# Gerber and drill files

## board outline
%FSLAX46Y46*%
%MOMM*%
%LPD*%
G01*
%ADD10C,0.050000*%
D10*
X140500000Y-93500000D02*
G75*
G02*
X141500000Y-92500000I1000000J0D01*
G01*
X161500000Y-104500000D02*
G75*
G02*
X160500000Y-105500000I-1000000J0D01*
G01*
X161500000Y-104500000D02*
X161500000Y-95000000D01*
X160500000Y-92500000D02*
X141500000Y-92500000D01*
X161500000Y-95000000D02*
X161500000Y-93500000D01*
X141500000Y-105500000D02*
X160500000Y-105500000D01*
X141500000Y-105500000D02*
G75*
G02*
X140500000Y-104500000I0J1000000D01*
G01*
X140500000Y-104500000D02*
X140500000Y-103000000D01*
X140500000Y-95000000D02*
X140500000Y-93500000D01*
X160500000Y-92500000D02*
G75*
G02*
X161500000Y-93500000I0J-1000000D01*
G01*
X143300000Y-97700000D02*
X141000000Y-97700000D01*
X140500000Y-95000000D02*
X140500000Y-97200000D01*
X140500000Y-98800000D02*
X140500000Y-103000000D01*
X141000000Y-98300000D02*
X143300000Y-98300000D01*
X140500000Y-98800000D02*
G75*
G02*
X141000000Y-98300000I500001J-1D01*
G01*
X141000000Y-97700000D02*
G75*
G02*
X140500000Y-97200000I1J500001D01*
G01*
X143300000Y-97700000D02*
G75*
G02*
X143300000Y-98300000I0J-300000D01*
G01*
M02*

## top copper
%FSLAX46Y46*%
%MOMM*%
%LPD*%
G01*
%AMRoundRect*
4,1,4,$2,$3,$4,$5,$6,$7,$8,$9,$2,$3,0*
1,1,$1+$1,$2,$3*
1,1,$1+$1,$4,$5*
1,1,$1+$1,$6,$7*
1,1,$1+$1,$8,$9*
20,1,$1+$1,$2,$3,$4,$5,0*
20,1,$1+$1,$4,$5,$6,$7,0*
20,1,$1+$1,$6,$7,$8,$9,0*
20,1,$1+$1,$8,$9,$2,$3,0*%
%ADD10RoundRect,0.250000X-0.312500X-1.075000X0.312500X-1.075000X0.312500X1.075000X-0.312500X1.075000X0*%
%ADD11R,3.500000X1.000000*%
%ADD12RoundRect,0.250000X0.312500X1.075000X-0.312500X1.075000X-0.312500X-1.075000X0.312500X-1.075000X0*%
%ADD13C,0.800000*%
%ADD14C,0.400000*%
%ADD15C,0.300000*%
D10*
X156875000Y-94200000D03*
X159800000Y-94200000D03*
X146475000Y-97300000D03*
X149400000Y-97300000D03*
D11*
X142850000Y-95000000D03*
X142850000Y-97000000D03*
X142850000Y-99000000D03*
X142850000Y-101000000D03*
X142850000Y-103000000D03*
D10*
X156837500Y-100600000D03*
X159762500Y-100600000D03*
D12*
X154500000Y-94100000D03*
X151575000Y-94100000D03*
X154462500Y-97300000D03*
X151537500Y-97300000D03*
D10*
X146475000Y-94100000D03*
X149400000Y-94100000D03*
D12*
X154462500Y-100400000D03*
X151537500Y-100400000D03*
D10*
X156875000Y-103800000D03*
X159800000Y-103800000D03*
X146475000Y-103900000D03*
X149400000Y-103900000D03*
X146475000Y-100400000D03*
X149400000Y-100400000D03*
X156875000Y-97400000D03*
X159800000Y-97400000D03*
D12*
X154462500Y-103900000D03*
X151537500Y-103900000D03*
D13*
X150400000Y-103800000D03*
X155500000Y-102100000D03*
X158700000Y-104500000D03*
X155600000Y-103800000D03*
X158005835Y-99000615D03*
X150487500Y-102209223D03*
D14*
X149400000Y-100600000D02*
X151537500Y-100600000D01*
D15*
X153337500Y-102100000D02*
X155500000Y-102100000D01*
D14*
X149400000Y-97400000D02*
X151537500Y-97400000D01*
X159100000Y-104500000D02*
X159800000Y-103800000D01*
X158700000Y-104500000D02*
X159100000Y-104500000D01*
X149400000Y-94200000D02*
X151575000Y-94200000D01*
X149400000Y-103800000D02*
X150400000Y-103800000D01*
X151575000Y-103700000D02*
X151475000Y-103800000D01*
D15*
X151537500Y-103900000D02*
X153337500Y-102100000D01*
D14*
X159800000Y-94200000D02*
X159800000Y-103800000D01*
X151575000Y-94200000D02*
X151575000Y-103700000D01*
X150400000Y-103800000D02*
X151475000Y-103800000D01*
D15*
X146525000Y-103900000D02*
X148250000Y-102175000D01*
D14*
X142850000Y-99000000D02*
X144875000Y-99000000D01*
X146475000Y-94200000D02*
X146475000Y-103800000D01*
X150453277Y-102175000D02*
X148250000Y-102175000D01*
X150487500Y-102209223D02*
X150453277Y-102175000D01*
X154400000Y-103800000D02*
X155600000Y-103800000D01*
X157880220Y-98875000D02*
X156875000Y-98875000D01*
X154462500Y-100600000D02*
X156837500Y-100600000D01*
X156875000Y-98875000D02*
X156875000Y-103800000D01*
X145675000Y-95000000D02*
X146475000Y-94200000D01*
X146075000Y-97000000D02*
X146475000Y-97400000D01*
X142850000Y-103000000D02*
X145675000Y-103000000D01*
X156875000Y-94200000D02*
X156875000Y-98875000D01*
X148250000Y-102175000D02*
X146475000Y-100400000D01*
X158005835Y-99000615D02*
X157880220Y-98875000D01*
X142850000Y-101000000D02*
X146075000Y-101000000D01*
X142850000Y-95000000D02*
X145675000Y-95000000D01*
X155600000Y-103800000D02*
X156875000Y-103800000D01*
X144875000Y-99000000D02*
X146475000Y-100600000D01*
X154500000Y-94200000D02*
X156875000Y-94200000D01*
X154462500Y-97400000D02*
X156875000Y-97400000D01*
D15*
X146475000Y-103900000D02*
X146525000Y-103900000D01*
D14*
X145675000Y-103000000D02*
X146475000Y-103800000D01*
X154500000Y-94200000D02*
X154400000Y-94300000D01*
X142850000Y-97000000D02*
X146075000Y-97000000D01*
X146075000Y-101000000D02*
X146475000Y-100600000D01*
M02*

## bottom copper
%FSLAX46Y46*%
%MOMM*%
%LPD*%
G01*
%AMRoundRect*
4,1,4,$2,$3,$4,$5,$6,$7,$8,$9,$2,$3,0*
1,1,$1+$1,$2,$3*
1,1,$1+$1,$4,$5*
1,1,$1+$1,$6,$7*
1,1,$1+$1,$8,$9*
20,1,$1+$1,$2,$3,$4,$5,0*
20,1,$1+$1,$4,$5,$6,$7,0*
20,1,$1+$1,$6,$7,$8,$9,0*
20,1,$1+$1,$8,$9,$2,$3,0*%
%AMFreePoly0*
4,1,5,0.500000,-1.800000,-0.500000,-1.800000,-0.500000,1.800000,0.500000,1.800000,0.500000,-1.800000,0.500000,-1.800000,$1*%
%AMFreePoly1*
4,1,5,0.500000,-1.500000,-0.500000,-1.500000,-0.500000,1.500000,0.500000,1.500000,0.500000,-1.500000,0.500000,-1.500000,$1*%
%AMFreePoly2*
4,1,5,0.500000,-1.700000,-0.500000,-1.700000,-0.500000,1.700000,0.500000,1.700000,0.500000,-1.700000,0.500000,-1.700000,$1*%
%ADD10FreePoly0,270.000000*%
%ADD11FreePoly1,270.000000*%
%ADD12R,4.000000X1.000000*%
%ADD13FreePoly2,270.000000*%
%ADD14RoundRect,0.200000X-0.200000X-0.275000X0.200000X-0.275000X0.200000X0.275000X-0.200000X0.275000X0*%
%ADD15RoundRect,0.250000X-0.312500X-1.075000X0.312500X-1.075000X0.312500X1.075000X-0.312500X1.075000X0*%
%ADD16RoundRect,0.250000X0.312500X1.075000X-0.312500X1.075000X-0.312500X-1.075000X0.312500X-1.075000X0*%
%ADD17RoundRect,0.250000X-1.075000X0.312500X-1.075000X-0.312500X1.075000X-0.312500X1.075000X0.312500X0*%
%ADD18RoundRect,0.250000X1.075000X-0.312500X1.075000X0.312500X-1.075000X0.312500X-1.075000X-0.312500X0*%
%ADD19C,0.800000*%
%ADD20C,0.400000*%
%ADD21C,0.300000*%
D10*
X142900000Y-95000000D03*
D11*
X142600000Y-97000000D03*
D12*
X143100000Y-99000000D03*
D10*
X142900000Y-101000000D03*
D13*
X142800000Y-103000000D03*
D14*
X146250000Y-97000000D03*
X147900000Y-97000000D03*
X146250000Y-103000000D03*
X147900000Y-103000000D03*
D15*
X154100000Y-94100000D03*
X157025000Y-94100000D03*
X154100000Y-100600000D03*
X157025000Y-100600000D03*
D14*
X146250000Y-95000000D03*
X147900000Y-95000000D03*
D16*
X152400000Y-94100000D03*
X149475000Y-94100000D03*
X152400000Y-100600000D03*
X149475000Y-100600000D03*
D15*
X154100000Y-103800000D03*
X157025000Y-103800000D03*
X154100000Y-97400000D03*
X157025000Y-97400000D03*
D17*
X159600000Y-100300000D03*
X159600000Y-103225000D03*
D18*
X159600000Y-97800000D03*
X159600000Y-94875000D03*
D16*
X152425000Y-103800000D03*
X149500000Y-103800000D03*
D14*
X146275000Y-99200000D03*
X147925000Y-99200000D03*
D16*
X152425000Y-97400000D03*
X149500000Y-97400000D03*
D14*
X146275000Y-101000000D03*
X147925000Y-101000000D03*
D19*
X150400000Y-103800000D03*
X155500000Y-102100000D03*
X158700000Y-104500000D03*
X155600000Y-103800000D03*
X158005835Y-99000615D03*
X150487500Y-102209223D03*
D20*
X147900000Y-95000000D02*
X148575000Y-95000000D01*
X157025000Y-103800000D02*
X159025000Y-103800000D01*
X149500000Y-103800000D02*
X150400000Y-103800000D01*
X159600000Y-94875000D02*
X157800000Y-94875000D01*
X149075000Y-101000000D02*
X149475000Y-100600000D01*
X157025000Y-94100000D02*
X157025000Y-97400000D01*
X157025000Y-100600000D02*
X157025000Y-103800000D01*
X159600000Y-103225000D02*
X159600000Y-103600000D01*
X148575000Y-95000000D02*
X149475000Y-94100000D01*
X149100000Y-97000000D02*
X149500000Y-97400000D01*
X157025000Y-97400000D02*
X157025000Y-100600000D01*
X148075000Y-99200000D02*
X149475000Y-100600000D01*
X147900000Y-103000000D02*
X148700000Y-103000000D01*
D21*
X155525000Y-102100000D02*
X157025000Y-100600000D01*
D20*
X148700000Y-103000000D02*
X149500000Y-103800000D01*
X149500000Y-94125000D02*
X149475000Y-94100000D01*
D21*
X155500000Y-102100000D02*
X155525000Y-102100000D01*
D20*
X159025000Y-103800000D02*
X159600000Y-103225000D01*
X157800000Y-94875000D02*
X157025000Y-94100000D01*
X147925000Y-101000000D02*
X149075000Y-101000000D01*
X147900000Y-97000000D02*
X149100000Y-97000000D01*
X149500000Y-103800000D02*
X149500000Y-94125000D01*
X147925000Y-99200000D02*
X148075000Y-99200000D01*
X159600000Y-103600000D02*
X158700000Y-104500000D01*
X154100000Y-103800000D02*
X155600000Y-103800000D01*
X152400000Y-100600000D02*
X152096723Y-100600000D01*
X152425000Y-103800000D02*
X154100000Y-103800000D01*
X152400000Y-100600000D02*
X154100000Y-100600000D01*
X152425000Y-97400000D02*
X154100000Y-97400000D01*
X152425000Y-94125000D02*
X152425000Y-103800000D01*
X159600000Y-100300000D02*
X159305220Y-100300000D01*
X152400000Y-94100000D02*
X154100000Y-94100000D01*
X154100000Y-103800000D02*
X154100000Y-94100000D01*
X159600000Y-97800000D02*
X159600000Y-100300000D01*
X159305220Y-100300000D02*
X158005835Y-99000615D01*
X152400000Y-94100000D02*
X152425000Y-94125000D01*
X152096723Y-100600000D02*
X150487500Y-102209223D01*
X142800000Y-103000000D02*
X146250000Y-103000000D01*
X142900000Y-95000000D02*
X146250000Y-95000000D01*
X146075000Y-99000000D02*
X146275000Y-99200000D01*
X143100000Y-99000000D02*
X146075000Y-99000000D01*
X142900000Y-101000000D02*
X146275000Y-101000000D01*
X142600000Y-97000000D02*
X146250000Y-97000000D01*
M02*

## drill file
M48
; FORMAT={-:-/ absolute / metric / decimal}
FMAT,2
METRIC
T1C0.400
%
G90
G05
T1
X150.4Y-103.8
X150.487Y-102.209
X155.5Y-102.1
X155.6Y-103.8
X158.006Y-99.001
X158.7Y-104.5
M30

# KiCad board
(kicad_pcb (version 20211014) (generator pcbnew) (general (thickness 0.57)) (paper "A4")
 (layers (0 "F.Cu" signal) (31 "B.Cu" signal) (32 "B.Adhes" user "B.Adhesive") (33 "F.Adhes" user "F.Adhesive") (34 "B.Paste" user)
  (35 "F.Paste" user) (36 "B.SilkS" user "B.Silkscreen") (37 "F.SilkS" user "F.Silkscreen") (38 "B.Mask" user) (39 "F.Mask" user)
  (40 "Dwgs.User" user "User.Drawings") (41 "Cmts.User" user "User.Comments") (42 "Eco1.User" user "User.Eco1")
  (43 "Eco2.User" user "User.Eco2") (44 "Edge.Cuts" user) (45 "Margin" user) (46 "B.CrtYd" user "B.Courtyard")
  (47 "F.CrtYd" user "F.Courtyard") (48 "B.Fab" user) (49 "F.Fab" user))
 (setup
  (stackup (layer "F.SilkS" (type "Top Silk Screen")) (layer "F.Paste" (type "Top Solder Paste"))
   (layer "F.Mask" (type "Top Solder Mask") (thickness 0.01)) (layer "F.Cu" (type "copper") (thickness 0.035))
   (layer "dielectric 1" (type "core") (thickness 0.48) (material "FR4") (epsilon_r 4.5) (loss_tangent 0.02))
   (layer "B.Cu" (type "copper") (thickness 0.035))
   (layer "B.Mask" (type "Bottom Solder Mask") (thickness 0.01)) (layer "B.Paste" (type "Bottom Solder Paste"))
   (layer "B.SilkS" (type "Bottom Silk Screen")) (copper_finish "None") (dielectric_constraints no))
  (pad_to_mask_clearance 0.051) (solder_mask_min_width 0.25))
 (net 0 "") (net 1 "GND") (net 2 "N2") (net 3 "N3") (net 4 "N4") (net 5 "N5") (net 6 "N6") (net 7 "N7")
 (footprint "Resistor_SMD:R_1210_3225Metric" (layer "F.Cu") (at 158.3375 94.2)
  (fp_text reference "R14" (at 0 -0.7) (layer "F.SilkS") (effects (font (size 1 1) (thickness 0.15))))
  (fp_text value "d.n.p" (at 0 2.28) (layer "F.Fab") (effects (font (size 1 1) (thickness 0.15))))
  (pad "1" smd roundrect (at -1.4625 0) (size 1.125 2.65) (layers "F.Cu" "F.Paste" "F.Mask") (roundrect_rratio 0.222222) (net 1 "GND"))
  (pad "2" smd roundrect (at 1.4625 0) (size 1.125 2.65) (layers "F.Cu" "F.Paste" "F.Mask") (roundrect_rratio 0.222222) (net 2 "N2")))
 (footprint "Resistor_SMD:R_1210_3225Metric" (layer "F.Cu") (at 147.9375 97.3)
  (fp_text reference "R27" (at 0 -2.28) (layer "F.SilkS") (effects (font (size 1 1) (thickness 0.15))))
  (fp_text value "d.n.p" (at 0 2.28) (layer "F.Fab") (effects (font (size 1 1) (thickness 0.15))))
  (pad "1" smd roundrect (at -1.4625 0) (size 1.125 2.65) (layers "F.Cu" "F.Paste" "F.Mask") (roundrect_rratio 0.222222) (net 1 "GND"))
  (pad "2" smd roundrect (at 1.4625 0) (size 1.125 2.65) (layers "F.Cu" "F.Paste" "F.Mask") (roundrect_rratio 0.222222) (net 2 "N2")))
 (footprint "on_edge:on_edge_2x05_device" (layer "F.Cu") (at 140.5 99 -90)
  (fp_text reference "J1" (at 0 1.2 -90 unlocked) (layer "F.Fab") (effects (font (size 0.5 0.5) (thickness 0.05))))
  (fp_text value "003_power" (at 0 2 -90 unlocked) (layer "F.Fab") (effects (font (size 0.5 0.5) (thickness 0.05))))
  (fp_line (start -1.3 -2.8) (end -1.3 -0.5) (layer "Edge.Cuts") (width 0.05))
  (fp_line (start -4 0) (end -1.8 0) (layer "Edge.Cuts") (width 0.05))
  (fp_line (start -0.2 0) (end 4 0) (layer "Edge.Cuts") (width 0.05))
  (fp_line (start -0.7 -0.5) (end -0.7 -2.8) (layer "Edge.Cuts") (width 0.05))
  (fp_arc (start -0.2 0) (mid -0.553553 -0.146447) (end -0.7 -0.5) (layer "Edge.Cuts") (width 0.05))
  (fp_arc (start -1.3 -0.5) (mid -1.446447 -0.146447) (end -1.8 0) (layer "Edge.Cuts") (width 0.05))
  (fp_arc (start -1.3 -2.8) (mid -1 -3.1) (end -0.7 -2.8) (layer "Edge.Cuts") (width 0.05))
  (pad "1" smd rect (at -4 -2.35 90) (size 1 3.5) (layers "F.Cu" "F.Mask") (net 1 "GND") (zone_connect 0))
  (pad "2" smd rect (at -2 -2.35 270) (size 1 3.5) (layers "F.Cu" "F.Mask") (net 1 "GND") (zone_connect 0))
  (pad "3" smd rect (at 0 -2.35 270) (size 1 3.5) (layers "F.Cu" "F.Mask") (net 1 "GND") (zone_connect 0))
  (pad "4" smd rect (at 2 -2.35 90) (size 1 3.5) (layers "F.Cu" "F.Mask") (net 1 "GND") (zone_connect 0))
  (pad "5" smd rect (at 4 -2.35 90) (size 1 3.5) (layers "F.Cu" "F.Mask") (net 1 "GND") (zone_connect 0))
  (pad "6" smd custom (at -4 -2.4 270) (size 1 3.6) (layers "B.Cu" "B.Mask") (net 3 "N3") (zone_connect 0)
   (options (clearance outline) (anchor rect)) (primitives))
  (pad "7" smd custom (at -2 -2.1 270) (size 1 3) (layers "B.Cu" "B.Mask") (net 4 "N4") (zone_connect 0)
   (options (clearance outline) (anchor rect)) (primitives))
  (pad "8" smd rect (at 0 -2.6 270) (size 1 4) (layers "B.Cu" "B.Mask") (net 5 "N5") (zone_connect 0))
  (pad "9" smd custom (at 2 -2.4 270) (size 1 3.6) (layers "B.Cu" "B.Mask") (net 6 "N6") (zone_connect 0)
   (options (clearance outline) (anchor rect)) (primitives))
  (pad "10" smd custom (at 4 -2.3 270) (size 1 3.4) (layers "B.Cu" "B.Mask") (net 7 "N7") (zone_connect 0)
   (options (clearance outline) (anchor rect)) (primitives)))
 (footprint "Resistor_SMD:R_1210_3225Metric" (layer "F.Cu") (at 158.3 100.6)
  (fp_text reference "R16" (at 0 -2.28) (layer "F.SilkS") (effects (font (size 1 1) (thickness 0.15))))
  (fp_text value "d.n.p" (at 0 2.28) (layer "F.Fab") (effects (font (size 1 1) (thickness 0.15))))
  (pad "1" smd roundrect (at -1.4625 0) (size 1.125 2.65) (layers "F.Cu" "F.Paste" "F.Mask") (roundrect_rratio 0.222222) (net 1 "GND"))
  (pad "2" smd roundrect (at 1.4625 0) (size 1.125 2.65) (layers "F.Cu" "F.Paste" "F.Mask") (roundrect_rratio 0.222222) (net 2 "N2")))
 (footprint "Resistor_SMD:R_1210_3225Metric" (layer "F.Cu") (at 153.0375 94.1 180)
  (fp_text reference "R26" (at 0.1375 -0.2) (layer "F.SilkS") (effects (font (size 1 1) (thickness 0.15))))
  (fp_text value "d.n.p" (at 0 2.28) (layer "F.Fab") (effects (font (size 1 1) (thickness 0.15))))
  (pad "1" smd roundrect (at -1.4625 0 180) (size 1.125 2.65) (layers "F.Cu" "F.Paste" "F.Mask") (roundrect_rratio 0.222222) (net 1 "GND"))
  (pad "2" smd roundrect (at 1.4625 0 180) (size 1.125 2.65) (layers "F.Cu" "F.Paste" "F.Mask") (roundrect_rratio 0.222222) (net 2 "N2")))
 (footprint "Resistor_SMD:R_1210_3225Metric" (layer "F.Cu") (at 153 97.3 180)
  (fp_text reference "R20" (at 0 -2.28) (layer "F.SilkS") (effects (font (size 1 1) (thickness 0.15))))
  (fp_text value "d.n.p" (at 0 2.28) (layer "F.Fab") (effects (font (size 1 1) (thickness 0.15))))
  (pad "1" smd roundrect (at -1.4625 0 180) (size 1.125 2.65) (layers "F.Cu" "F.Paste" "F.Mask") (roundrect_rratio 0.222222) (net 1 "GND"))
  (pad "2" smd roundrect (at 1.4625 0 180) (size 1.125 2.65) (layers "F.Cu" "F.Paste" "F.Mask") (roundrect_rratio 0.222222) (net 2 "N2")))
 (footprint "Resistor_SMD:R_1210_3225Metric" (layer "F.Cu") (at 147.9375 94.1)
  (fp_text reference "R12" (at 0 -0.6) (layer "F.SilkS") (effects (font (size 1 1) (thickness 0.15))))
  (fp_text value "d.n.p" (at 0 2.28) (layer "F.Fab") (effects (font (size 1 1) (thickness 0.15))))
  (pad "1" smd roundrect (at -1.4625 0) (size 1.125 2.65) (layers "F.Cu" "F.Paste" "F.Mask") (roundrect_rratio 0.222222) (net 1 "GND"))
  (pad "2" smd roundrect (at 1.4625 0) (size 1.125 2.65) (layers "F.Cu" "F.Paste" "F.Mask") (roundrect_rratio 0.222222) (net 2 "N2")))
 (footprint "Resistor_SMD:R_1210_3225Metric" (layer "F.Cu") (at 153 100.4 180)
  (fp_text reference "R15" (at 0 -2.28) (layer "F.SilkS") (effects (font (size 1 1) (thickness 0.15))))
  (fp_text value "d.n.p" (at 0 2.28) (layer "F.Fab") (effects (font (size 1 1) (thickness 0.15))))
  (pad "1" smd roundrect (at -1.4625 0 180) (size 1.125 2.65) (layers "F.Cu" "F.Paste" "F.Mask") (roundrect_rratio 0.222222) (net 1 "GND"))
  (pad "2" smd roundrect (at 1.4625 0 180) (size 1.125 2.65) (layers "F.Cu" "F.Paste" "F.Mask") (roundrect_rratio 0.222222) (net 2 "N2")))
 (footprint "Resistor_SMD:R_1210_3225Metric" (layer "F.Cu") (at 158.3375 103.8)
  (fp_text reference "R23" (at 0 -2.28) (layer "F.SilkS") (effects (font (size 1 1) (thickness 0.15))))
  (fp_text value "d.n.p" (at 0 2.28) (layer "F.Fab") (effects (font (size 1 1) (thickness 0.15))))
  (pad "1" smd roundrect (at -1.4625 0) (size 1.125 2.65) (layers "F.Cu" "F.Paste" "F.Mask") (roundrect_rratio 0.222222) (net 1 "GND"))
  (pad "2" smd roundrect (at 1.4625 0) (size 1.125 2.65) (layers "F.Cu" "F.Paste" "F.Mask") (roundrect_rratio 0.222222) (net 2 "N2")))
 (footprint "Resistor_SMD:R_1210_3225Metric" (layer "F.Cu") (at 147.9375 103.9)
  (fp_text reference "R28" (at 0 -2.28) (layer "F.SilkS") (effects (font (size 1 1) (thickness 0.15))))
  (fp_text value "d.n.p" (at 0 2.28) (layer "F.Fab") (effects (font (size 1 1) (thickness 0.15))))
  (pad "1" smd roundrect (at -1.4625 0) (size 1.125 2.65) (layers "F.Cu" "F.Paste" "F.Mask") (roundrect_rratio 0.222222) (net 1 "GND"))
  (pad "2" smd roundrect (at 1.4625 0) (size 1.125 2.65) (layers "F.Cu" "F.Paste" "F.Mask") (roundrect_rratio 0.222222) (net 2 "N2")))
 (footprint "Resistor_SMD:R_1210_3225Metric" (layer "F.Cu") (at 147.9375 100.4)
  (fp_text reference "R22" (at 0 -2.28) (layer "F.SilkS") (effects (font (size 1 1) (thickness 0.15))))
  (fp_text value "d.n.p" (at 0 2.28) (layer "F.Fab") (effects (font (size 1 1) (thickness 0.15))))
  (pad "1" smd roundrect (at -1.4625 0) (size 1.125 2.65) (layers "F.Cu" "F.Paste" "F.Mask") (roundrect_rratio 0.222222) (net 1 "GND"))
  (pad "2" smd roundrect (at 1.4625 0) (size 1.125 2.65) (layers "F.Cu" "F.Paste" "F.Mask") (roundrect_rratio 0.222222) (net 2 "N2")))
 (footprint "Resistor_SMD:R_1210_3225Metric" (layer "F.Cu") (at 158.3375 97.4)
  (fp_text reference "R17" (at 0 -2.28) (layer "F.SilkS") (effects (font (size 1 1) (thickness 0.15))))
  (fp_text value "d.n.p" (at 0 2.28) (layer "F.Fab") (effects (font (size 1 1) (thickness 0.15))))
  (pad "1" smd roundrect (at -1.4625 0) (size 1.125 2.65) (layers "F.Cu" "F.Paste" "F.Mask") (roundrect_rratio 0.222222) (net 1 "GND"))
  (pad "2" smd roundrect (at 1.4625 0) (size 1.125 2.65) (layers "F.Cu" "F.Paste" "F.Mask") (roundrect_rratio 0.222222) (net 2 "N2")))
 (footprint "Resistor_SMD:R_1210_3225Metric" (layer "F.Cu") (at 153 103.9 180)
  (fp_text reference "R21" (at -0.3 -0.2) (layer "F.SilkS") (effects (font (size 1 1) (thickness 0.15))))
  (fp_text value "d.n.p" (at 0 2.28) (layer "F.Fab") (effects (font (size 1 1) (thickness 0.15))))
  (pad "1" smd roundrect (at -1.4625 0 180) (size 1.125 2.65) (layers "F.Cu" "F.Paste" "F.Mask") (roundrect_rratio 0.222222) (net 1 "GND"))
  (pad "2" smd roundrect (at 1.4625 0 180) (size 1.125 2.65) (layers "F.Cu" "F.Paste" "F.Mask") (roundrect_rratio 0.222222) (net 2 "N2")))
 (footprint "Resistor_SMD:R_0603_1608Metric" (layer "B.Cu") (at 147.075 97)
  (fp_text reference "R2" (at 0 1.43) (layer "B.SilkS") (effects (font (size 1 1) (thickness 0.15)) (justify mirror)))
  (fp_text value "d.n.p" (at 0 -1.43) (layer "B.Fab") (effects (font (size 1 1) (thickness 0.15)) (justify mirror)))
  (pad "1" smd roundrect (at -0.825 0) (size 0.8 0.95) (layers "B.Cu" "B.Paste" "B.Mask") (roundrect_rratio 0.25) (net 4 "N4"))
  (pad "2" smd roundrect (at 0.825 0) (size 0.8 0.95) (layers "B.Cu" "B.Paste" "B.Mask") (roundrect_rratio 0.25) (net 2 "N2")))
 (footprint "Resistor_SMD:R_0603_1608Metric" (layer "B.Cu") (at 147.075 103)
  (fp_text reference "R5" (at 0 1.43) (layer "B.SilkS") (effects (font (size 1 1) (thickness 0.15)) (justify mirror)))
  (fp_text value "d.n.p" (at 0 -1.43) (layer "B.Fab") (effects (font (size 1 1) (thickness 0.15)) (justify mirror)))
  (pad "1" smd roundrect (at -0.825 0) (size 0.8 0.95) (layers "B.Cu" "B.Paste" "B.Mask") (roundrect_rratio 0.25) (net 7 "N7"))
  (pad "2" smd roundrect (at 0.825 0) (size 0.8 0.95) (layers "B.Cu" "B.Paste" "B.Mask") (roundrect_rratio 0.25) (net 2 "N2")))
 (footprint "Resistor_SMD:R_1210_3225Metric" (layer "B.Cu") (at 155.5625 94.1)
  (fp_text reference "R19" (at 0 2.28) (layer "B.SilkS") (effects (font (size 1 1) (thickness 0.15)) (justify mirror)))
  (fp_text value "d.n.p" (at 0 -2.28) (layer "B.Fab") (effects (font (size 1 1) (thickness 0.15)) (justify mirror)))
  (pad "1" smd roundrect (at -1.4625 0) (size 1.125 2.65) (layers "B.Cu" "B.Paste" "B.Mask") (roundrect_rratio 0.222222) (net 1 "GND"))
  (pad "2" smd roundrect (at 1.4625 0) (size 1.125 2.65) (layers "B.Cu" "B.Paste" "B.Mask") (roundrect_rratio 0.222222) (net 2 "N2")))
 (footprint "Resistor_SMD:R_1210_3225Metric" (layer "B.Cu") (at 155.5625 100.6)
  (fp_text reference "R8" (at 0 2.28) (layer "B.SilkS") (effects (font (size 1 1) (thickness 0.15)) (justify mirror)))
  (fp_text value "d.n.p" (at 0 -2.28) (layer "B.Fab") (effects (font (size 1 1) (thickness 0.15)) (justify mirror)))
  (pad "1" smd roundrect (at -1.4625 0) (size 1.125 2.65) (layers "B.Cu" "B.Paste" "B.Mask") (roundrect_rratio 0.222222) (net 1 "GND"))
  (pad "2" smd roundrect (at 1.4625 0) (size 1.125 2.65) (layers "B.Cu" "B.Paste" "B.Mask") (roundrect_rratio 0.222222) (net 2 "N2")))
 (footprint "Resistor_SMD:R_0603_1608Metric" (layer "B.Cu") (at 147.075 95)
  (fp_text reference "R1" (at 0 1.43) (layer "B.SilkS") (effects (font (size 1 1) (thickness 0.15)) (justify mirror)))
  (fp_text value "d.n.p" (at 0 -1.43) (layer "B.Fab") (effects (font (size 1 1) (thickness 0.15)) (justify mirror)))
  (pad "1" smd roundrect (at -0.825 0) (size 0.8 0.95) (layers "B.Cu" "B.Paste" "B.Mask") (roundrect_rratio 0.25) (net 3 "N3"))
  (pad "2" smd roundrect (at 0.825 0) (size 0.8 0.95) (layers "B.Cu" "B.Paste" "B.Mask") (roundrect_rratio 0.25) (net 2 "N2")))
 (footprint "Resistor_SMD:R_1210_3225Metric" (layer "B.Cu") (at 150.9375 94.1 180)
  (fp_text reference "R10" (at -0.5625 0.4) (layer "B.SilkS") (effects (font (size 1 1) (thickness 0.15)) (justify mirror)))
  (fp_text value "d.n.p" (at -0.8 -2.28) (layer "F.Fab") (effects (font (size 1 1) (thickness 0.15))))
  (pad "1" smd roundrect (at -1.4625 0 180) (size 1.125 2.65) (layers "B.Cu" "B.Paste" "B.Mask") (roundrect_rratio 0.222222) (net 1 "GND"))
  (pad "2" smd roundrect (at 1.4625 0 180) (size 1.125 2.65) (layers "B.Cu" "B.Paste" "B.Mask") (roundrect_rratio 0.222222) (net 2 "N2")))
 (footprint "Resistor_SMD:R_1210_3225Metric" (layer "B.Cu") (at 150.9375 100.6 180)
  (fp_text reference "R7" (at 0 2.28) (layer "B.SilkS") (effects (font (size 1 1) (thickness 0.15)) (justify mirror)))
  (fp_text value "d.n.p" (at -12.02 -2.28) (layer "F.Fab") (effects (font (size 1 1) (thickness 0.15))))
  (pad "1" smd roundrect (at -1.4625 0 180) (size 1.125 2.65) (layers "B.Cu" "B.Paste" "B.Mask") (roundrect_rratio 0.222222) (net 1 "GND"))
  (pad "2" smd roundrect (at 1.4625 0 180) (size 1.125 2.65) (layers "B.Cu" "B.Paste" "B.Mask") (roundrect_rratio 0.222222) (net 2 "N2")))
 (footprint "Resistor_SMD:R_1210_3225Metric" (layer "B.Cu") (at 155.5625 103.8)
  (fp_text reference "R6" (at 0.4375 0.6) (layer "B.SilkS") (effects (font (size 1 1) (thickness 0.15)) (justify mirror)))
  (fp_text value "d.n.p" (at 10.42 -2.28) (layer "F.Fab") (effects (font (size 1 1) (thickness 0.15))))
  (pad "1" smd roundrect (at -1.4625 0) (size 1.125 2.65) (layers "B.Cu" "B.Paste" "B.Mask") (roundrect_rratio 0.222222) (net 1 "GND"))
  (pad "2" smd roundrect (at 1.4625 0) (size 1.125 2.65) (layers "B.Cu" "B.Paste" "B.Mask") (roundrect_rratio 0.222222) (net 2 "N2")))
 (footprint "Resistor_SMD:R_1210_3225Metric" (layer "B.Cu") (at 155.5625 97.4)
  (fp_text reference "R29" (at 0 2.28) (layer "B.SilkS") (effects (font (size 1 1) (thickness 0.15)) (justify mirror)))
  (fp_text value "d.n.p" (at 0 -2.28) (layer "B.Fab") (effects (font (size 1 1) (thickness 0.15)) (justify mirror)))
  (pad "1" smd roundrect (at -1.4625 0) (size 1.125 2.65) (layers "B.Cu" "B.Paste" "B.Mask") (roundrect_rratio 0.222222) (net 1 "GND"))
  (pad "2" smd roundrect (at 1.4625 0) (size 1.125 2.65) (layers "B.Cu" "B.Paste" "B.Mask") (roundrect_rratio 0.222222) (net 2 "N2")))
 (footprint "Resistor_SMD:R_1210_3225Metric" (layer "B.Cu") (at 159.6 101.7625 -90)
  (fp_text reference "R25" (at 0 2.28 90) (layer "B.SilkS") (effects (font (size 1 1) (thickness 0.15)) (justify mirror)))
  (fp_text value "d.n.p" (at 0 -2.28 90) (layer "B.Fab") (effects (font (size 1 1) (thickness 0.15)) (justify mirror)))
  (pad "1" smd roundrect (at -1.4625 0 270) (size 1.125 2.65) (layers "B.Cu" "B.Paste" "B.Mask") (roundrect_rratio 0.222222) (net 1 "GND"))
  (pad "2" smd roundrect (at 1.4625 0 270) (size 1.125 2.65) (layers "B.Cu" "B.Paste" "B.Mask") (roundrect_rratio 0.222222) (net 2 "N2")))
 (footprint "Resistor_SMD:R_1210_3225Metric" (layer "B.Cu") (at 159.6 96.3375 90)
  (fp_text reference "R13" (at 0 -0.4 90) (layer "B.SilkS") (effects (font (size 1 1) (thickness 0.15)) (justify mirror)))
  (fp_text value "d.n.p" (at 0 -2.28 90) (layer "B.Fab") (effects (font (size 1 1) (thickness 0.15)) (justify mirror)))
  (pad "1" smd roundrect (at -1.4625 0 90) (size 1.125 2.65) (layers "B.Cu" "B.Paste" "B.Mask") (roundrect_rratio 0.222222) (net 1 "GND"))
  (pad "2" smd roundrect (at 1.4625 0 90) (size 1.125 2.65) (layers "B.Cu" "B.Paste" "B.Mask") (roundrect_rratio 0.222222) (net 2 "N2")))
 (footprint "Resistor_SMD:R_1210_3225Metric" (layer "B.Cu") (at 150.9625 103.8 180)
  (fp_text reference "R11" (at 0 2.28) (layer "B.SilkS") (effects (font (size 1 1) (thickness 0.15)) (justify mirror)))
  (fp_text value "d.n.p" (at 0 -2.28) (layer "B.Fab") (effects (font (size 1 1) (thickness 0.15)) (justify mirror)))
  (pad "1" smd roundrect (at -1.4625 0 180) (size 1.125 2.65) (layers "B.Cu" "B.Paste" "B.Mask") (roundrect_rratio 0.222222) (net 1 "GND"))
  (pad "2" smd roundrect (at 1.4625 0 180) (size 1.125 2.65) (layers "B.Cu" "B.Paste" "B.Mask") (roundrect_rratio 0.222222) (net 2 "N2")))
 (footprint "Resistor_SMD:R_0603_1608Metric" (layer "B.Cu") (at 147.1 99.2)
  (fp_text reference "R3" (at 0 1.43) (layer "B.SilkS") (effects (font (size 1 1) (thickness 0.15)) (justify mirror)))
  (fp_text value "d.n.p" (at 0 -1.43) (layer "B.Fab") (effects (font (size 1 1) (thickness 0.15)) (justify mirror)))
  (pad "1" smd roundrect (at -0.825 0) (size 0.8 0.95) (layers "B.Cu" "B.Paste" "B.Mask") (roundrect_rratio 0.25) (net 5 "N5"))
  (pad "2" smd roundrect (at 0.825 0) (size 0.8 0.95) (layers "B.Cu" "B.Paste" "B.Mask") (roundrect_rratio 0.25) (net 2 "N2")))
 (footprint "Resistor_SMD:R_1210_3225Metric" (layer "B.Cu") (at 150.9625 97.4 180)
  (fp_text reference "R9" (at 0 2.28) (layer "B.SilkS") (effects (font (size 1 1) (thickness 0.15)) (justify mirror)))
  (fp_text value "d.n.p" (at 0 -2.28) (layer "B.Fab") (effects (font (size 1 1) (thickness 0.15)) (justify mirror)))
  (pad "1" smd roundrect (at -1.4625 0 180) (size 1.125 2.65) (layers "B.Cu" "B.Paste" "B.Mask") (roundrect_rratio 0.222222) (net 1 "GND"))
  (pad "2" smd roundrect (at 1.4625 0 180) (size 1.125 2.65) (layers "B.Cu" "B.Paste" "B.Mask") (roundrect_rratio 0.222222) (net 2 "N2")))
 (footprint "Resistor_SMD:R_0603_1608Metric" (layer "B.Cu") (at 147.1 101)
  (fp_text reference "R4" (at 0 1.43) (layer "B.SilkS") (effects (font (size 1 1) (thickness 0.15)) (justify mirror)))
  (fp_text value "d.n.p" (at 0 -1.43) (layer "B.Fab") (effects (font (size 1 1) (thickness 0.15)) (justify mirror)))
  (pad "1" smd roundrect (at -0.825 0) (size 0.8 0.95) (layers "B.Cu" "B.Paste" "B.Mask") (roundrect_rratio 0.25) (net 6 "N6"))
  (pad "2" smd roundrect (at 0.825 0) (size 0.8 0.95) (layers "B.Cu" "B.Paste" "B.Mask") (roundrect_rratio 0.25) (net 2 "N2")))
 (gr_arc (start 140.5 93.5) (mid 140.792893 92.792893) (end 141.5 92.5) (layer "Edge.Cuts") (width 0.05))
 (gr_arc (start 161.5 104.5) (mid 161.207107 105.207107) (end 160.5 105.5) (layer "Edge.Cuts") (width 0.05))
 (gr_line (start 161.5 104.5) (end 161.5 95) (layer "Edge.Cuts") (width 0.05))
 (gr_line (start 160.5 92.5) (end 141.5 92.5) (layer "Edge.Cuts") (width 0.05))
 (gr_line (start 161.5 95) (end 161.5 93.5) (layer "Edge.Cuts") (width 0.05))
 (gr_line (start 141.5 105.5) (end 160.5 105.5) (layer "Edge.Cuts") (width 0.05))
 (gr_arc (start 141.5 105.5) (mid 140.792893 105.207107) (end 140.5 104.5) (layer "Edge.Cuts") (width 0.05))
 (gr_line (start 140.5 104.5) (end 140.5 103) (layer "Edge.Cuts") (width 0.05))
 (gr_line (start 140.5 95) (end 140.5 93.5) (layer "Edge.Cuts") (width 0.05))
 (gr_arc (start 160.5 92.5) (mid 161.207107 92.792893) (end 161.5 93.5) (layer "Edge.Cuts") (width 0.05))
 (segment (start 149.4 100.6) (end 151.5375 100.6) (width 0.4) (layer "F.Cu") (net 2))
 (segment (start 153.3375 102.1) (end 155.5 102.1) (width 0.3) (layer "F.Cu") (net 2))
 (segment (start 149.4 97.4) (end 151.5375 97.4) (width 0.4) (layer "F.Cu") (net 2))
 (segment (start 159.1 104.5) (end 159.8 103.8) (width 0.4) (layer "F.Cu") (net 2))
 (segment (start 158.7 104.5) (end 159.1 104.5) (width 0.4) (layer "F.Cu") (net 2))
 (segment (start 149.4 94.2) (end 151.575 94.2) (width 0.4) (layer "F.Cu") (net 2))
 (segment (start 149.4 103.8) (end 150.4 103.8) (width 0.4) (layer "F.Cu") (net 2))
 (segment (start 151.575 103.7) (end 151.475 103.8) (width 0.4) (layer "F.Cu") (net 2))
 (segment (start 151.5375 103.9) (end 153.3375 102.1) (width 0.3) (layer "F.Cu") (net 2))
 (segment (start 159.8 94.2) (end 159.8 103.8) (width 0.4) (layer "F.Cu") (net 2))
 (segment (start 151.575 94.2) (end 151.575 103.7) (width 0.4) (layer "F.Cu") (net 2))
 (segment (start 150.4 103.8) (end 151.475 103.8) (width 0.4) (layer "F.Cu") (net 2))
 (via (at 150.4 103.8) (size 0.8) (drill 0.4) (layers "F.Cu" "B.Cu") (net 2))
 (via (at 155.5 102.1) (size 0.8) (drill 0.4) (layers "F.Cu" "B.Cu") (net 2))
 (via (at 158.7 104.5) (size 0.8) (drill 0.4) (layers "F.Cu" "B.Cu") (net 2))
 (segment (start 147.9 95) (end 148.575 95) (width 0.4) (layer "B.Cu") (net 2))
 (segment (start 157.025 103.8) (end 159.025 103.8) (width 0.4) (layer "B.Cu") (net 2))
 (segment (start 149.5 103.8) (end 150.4 103.8) (width 0.4) (layer "B.Cu") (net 2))
 (segment (start 159.6 94.875) (end 157.8 94.875) (width 0.4) (layer "B.Cu") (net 2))
 (segment (start 149.075 101) (end 149.475 100.6) (width 0.4) (layer "B.Cu") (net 2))
 (segment (start 157.025 94.1) (end 157.025 97.4) (width 0.4) (layer "B.Cu") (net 2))
 (segment (start 157.025 100.6) (end 157.025 103.8) (width 0.4) (layer "B.Cu") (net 2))
 (segment (start 159.6 103.225) (end 159.6 103.6) (width 0.4) (layer "B.Cu") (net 2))
 (segment (start 148.575 95) (end 149.475 94.1) (width 0.4) (layer "B.Cu") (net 2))
 (segment (start 149.1 97) (end 149.5 97.4) (width 0.4) (layer "B.Cu") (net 2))
 (segment (start 157.025 97.4) (end 157.025 100.6) (width 0.4) (layer "B.Cu") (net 2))
 (segment (start 148.075 99.2) (end 149.475 100.6) (width 0.4) (layer "B.Cu") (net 2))
 (segment (start 147.9 103) (end 148.7 103) (width 0.4) (layer "B.Cu") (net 2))
 (segment (start 155.525 102.1) (end 157.025 100.6) (width 0.3) (layer "B.Cu") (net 2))
 (segment (start 148.7 103) (end 149.5 103.8) (width 0.4) (layer "B.Cu") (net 2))
 (segment (start 149.5 94.125) (end 149.475 94.1) (width 0.4) (layer "B.Cu") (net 2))
 (segment (start 155.5 102.1) (end 155.525 102.1) (width 0.3) (layer "B.Cu") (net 2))
 (segment (start 159.025 103.8) (end 159.6 103.225) (width 0.4) (layer "B.Cu") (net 2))
 (segment (start 157.8 94.875) (end 157.025 94.1) (width 0.4) (layer "B.Cu") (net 2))
 (segment (start 147.925 101) (end 149.075 101) (width 0.4) (layer "B.Cu") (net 2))
 (segment (start 147.9 97) (end 149.1 97) (width 0.4) (layer "B.Cu") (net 2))
 (segment (start 149.5 103.8) (end 149.5 94.125) (width 0.4) (layer "B.Cu") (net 2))
 (segment (start 147.925 99.2) (end 148.075 99.2) (width 0.4) (layer "B.Cu") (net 2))
 (segment (start 159.6 103.6) (end 158.7 104.5) (width 0.4) (layer "B.Cu") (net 2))
 (segment (start 146.525 103.9) (end 148.25 102.175) (width 0.3) (layer "F.Cu") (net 1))
 (segment (start 142.85 99) (end 144.875 99) (width 0.4) (layer "F.Cu") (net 1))
 (segment (start 146.475 94.2) (end 146.475 103.8) (width 0.4) (layer "F.Cu") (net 1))
 (segment (start 150.453277 102.175) (end 148.25 102.175) (width 0.4) (layer "F.Cu") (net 1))
 (segment (start 150.4875 102.209223) (end 150.453277 102.175) (width 0.4) (layer "F.Cu") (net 1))
 (segment (start 154.4 103.8) (end 155.6 103.8) (width 0.4) (layer "F.Cu") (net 1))
 (segment (start 157.88022 98.875) (end 156.875 98.875) (width 0.4) (layer "F.Cu") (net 1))
 (segment (start 154.4625 100.6) (end 156.8375 100.6) (width 0.4) (layer "F.Cu") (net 1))
 (segment (start 156.875 98.875) (end 156.875 103.8) (width 0.4) (layer "F.Cu") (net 1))
 (segment (start 145.675 95) (end 146.475 94.2) (width 0.4) (layer "F.Cu") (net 1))
 (segment (start 146.075 97) (end 146.475 97.4) (width 0.4) (layer "F.Cu") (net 1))
 (segment (start 142.85 103) (end 145.675 103) (width 0.4) (layer "F.Cu") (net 1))
 (segment (start 156.875 94.2) (end 156.875 98.875) (width 0.4) (layer "F.Cu") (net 1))
 (segment (start 148.25 102.175) (end 146.475 100.4) (width 0.4) (layer "F.Cu") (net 1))
 (segment (start 158.005835 99.000615) (end 157.88022 98.875) (width 0.4) (layer "F.Cu") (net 1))
 (segment (start 142.85 101) (end 146.075 101) (width 0.4) (layer "F.Cu") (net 1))
 (segment (start 142.85 95) (end 145.675 95) (width 0.4) (layer "F.Cu") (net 1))
 (segment (start 155.6 103.8) (end 156.875 103.8) (width 0.4) (layer "F.Cu") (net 1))
 (segment (start 144.875 99) (end 146.475 100.6) (width 0.4) (layer "F.Cu") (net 1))
 (segment (start 154.5 94.2) (end 156.875 94.2) (width 0.4) (layer "F.Cu") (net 1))
 (segment (start 154.4625 97.4) (end 156.875 97.4) (width 0.4) (layer "F.Cu") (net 1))
 (segment (start 146.475 103.9) (end 146.525 103.9) (width 0.3) (layer "F.Cu") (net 1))
 (segment (start 145.675 103) (end 146.475 103.8) (width 0.4) (layer "F.Cu") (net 1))
 (segment (start 154.5 94.2) (end 154.4 94.3) (width 0.4) (layer "F.Cu") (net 1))
 (segment (start 142.85 97) (end 146.075 97) (width 0.4) (layer "F.Cu") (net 1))
 (segment (start 146.075 101) (end 146.475 100.6) (width 0.4) (layer "F.Cu") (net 1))
 (via (at 155.6 103.8) (size 0.8) (drill 0.4) (layers "F.Cu" "B.Cu") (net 1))
 (via (at 158.005835 99.000615) (size 0.8) (drill 0.4) (layers "F.Cu" "B.Cu") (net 1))
 (via (at 150.4875 102.209223) (size 0.8) (drill 0.4) (layers "F.Cu" "B.Cu") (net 1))
 (segment (start 154.1 103.8) (end 155.6 103.8) (width 0.4) (layer "B.Cu") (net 1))
 (segment (start 152.4 100.6) (end 152.096723 100.6) (width 0.4) (layer "B.Cu") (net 1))
 (segment (start 152.425 103.8) (end 154.1 103.8) (width 0.4) (layer "B.Cu") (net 1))
 (segment (start 152.4 100.6) (end 154.1 100.6) (width 0.4) (layer "B.Cu") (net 1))
 (segment (start 152.425 97.4) (end 154.1 97.4) (width 0.4) (layer "B.Cu") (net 1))
 (segment (start 152.425 94.125) (end 152.425 103.8) (width 0.4) (layer "B.Cu") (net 1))
 (segment (start 159.6 100.3) (end 159.30522 100.3) (width 0.4) (layer "B.Cu") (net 1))
 (segment (start 152.4 94.1) (end 154.1 94.1) (width 0.4) (layer "B.Cu") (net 1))
 (segment (start 154.1 103.8) (end 154.1 94.1) (width 0.4) (layer "B.Cu") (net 1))
 (segment (start 159.6 97.8) (end 159.6 100.3) (width 0.4) (layer "B.Cu") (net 1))
 (segment (start 159.30522 100.3) (end 158.005835 99.000615) (width 0.4) (layer "B.Cu") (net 1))
 (segment (start 152.4 94.1) (end 152.425 94.125) (width 0.4) (layer "B.Cu") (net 1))
 (segment (start 152.096723 100.6) (end 150.4875 102.209223) (width 0.4) (layer "B.Cu") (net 1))
 (segment (start 142.8 103) (end 146.25 103) (width 0.4) (layer "B.Cu") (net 7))
 (segment (start 142.9 95) (end 146.25 95) (width 0.4) (layer "B.Cu") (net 3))
 (segment (start 146.075 99) (end 146.275 99.2) (width 0.4) (layer "B.Cu") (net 5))
 (segment (start 143.1 99) (end 146.075 99) (width 0.4) (layer "B.Cu") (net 5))
 (segment (start 142.9 101) (end 146.275 101) (width 0.4) (layer "B.Cu") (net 6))
 (segment (start 142.6 97) (end 146.25 97) (width 0.4) (layer "B.Cu") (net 4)))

